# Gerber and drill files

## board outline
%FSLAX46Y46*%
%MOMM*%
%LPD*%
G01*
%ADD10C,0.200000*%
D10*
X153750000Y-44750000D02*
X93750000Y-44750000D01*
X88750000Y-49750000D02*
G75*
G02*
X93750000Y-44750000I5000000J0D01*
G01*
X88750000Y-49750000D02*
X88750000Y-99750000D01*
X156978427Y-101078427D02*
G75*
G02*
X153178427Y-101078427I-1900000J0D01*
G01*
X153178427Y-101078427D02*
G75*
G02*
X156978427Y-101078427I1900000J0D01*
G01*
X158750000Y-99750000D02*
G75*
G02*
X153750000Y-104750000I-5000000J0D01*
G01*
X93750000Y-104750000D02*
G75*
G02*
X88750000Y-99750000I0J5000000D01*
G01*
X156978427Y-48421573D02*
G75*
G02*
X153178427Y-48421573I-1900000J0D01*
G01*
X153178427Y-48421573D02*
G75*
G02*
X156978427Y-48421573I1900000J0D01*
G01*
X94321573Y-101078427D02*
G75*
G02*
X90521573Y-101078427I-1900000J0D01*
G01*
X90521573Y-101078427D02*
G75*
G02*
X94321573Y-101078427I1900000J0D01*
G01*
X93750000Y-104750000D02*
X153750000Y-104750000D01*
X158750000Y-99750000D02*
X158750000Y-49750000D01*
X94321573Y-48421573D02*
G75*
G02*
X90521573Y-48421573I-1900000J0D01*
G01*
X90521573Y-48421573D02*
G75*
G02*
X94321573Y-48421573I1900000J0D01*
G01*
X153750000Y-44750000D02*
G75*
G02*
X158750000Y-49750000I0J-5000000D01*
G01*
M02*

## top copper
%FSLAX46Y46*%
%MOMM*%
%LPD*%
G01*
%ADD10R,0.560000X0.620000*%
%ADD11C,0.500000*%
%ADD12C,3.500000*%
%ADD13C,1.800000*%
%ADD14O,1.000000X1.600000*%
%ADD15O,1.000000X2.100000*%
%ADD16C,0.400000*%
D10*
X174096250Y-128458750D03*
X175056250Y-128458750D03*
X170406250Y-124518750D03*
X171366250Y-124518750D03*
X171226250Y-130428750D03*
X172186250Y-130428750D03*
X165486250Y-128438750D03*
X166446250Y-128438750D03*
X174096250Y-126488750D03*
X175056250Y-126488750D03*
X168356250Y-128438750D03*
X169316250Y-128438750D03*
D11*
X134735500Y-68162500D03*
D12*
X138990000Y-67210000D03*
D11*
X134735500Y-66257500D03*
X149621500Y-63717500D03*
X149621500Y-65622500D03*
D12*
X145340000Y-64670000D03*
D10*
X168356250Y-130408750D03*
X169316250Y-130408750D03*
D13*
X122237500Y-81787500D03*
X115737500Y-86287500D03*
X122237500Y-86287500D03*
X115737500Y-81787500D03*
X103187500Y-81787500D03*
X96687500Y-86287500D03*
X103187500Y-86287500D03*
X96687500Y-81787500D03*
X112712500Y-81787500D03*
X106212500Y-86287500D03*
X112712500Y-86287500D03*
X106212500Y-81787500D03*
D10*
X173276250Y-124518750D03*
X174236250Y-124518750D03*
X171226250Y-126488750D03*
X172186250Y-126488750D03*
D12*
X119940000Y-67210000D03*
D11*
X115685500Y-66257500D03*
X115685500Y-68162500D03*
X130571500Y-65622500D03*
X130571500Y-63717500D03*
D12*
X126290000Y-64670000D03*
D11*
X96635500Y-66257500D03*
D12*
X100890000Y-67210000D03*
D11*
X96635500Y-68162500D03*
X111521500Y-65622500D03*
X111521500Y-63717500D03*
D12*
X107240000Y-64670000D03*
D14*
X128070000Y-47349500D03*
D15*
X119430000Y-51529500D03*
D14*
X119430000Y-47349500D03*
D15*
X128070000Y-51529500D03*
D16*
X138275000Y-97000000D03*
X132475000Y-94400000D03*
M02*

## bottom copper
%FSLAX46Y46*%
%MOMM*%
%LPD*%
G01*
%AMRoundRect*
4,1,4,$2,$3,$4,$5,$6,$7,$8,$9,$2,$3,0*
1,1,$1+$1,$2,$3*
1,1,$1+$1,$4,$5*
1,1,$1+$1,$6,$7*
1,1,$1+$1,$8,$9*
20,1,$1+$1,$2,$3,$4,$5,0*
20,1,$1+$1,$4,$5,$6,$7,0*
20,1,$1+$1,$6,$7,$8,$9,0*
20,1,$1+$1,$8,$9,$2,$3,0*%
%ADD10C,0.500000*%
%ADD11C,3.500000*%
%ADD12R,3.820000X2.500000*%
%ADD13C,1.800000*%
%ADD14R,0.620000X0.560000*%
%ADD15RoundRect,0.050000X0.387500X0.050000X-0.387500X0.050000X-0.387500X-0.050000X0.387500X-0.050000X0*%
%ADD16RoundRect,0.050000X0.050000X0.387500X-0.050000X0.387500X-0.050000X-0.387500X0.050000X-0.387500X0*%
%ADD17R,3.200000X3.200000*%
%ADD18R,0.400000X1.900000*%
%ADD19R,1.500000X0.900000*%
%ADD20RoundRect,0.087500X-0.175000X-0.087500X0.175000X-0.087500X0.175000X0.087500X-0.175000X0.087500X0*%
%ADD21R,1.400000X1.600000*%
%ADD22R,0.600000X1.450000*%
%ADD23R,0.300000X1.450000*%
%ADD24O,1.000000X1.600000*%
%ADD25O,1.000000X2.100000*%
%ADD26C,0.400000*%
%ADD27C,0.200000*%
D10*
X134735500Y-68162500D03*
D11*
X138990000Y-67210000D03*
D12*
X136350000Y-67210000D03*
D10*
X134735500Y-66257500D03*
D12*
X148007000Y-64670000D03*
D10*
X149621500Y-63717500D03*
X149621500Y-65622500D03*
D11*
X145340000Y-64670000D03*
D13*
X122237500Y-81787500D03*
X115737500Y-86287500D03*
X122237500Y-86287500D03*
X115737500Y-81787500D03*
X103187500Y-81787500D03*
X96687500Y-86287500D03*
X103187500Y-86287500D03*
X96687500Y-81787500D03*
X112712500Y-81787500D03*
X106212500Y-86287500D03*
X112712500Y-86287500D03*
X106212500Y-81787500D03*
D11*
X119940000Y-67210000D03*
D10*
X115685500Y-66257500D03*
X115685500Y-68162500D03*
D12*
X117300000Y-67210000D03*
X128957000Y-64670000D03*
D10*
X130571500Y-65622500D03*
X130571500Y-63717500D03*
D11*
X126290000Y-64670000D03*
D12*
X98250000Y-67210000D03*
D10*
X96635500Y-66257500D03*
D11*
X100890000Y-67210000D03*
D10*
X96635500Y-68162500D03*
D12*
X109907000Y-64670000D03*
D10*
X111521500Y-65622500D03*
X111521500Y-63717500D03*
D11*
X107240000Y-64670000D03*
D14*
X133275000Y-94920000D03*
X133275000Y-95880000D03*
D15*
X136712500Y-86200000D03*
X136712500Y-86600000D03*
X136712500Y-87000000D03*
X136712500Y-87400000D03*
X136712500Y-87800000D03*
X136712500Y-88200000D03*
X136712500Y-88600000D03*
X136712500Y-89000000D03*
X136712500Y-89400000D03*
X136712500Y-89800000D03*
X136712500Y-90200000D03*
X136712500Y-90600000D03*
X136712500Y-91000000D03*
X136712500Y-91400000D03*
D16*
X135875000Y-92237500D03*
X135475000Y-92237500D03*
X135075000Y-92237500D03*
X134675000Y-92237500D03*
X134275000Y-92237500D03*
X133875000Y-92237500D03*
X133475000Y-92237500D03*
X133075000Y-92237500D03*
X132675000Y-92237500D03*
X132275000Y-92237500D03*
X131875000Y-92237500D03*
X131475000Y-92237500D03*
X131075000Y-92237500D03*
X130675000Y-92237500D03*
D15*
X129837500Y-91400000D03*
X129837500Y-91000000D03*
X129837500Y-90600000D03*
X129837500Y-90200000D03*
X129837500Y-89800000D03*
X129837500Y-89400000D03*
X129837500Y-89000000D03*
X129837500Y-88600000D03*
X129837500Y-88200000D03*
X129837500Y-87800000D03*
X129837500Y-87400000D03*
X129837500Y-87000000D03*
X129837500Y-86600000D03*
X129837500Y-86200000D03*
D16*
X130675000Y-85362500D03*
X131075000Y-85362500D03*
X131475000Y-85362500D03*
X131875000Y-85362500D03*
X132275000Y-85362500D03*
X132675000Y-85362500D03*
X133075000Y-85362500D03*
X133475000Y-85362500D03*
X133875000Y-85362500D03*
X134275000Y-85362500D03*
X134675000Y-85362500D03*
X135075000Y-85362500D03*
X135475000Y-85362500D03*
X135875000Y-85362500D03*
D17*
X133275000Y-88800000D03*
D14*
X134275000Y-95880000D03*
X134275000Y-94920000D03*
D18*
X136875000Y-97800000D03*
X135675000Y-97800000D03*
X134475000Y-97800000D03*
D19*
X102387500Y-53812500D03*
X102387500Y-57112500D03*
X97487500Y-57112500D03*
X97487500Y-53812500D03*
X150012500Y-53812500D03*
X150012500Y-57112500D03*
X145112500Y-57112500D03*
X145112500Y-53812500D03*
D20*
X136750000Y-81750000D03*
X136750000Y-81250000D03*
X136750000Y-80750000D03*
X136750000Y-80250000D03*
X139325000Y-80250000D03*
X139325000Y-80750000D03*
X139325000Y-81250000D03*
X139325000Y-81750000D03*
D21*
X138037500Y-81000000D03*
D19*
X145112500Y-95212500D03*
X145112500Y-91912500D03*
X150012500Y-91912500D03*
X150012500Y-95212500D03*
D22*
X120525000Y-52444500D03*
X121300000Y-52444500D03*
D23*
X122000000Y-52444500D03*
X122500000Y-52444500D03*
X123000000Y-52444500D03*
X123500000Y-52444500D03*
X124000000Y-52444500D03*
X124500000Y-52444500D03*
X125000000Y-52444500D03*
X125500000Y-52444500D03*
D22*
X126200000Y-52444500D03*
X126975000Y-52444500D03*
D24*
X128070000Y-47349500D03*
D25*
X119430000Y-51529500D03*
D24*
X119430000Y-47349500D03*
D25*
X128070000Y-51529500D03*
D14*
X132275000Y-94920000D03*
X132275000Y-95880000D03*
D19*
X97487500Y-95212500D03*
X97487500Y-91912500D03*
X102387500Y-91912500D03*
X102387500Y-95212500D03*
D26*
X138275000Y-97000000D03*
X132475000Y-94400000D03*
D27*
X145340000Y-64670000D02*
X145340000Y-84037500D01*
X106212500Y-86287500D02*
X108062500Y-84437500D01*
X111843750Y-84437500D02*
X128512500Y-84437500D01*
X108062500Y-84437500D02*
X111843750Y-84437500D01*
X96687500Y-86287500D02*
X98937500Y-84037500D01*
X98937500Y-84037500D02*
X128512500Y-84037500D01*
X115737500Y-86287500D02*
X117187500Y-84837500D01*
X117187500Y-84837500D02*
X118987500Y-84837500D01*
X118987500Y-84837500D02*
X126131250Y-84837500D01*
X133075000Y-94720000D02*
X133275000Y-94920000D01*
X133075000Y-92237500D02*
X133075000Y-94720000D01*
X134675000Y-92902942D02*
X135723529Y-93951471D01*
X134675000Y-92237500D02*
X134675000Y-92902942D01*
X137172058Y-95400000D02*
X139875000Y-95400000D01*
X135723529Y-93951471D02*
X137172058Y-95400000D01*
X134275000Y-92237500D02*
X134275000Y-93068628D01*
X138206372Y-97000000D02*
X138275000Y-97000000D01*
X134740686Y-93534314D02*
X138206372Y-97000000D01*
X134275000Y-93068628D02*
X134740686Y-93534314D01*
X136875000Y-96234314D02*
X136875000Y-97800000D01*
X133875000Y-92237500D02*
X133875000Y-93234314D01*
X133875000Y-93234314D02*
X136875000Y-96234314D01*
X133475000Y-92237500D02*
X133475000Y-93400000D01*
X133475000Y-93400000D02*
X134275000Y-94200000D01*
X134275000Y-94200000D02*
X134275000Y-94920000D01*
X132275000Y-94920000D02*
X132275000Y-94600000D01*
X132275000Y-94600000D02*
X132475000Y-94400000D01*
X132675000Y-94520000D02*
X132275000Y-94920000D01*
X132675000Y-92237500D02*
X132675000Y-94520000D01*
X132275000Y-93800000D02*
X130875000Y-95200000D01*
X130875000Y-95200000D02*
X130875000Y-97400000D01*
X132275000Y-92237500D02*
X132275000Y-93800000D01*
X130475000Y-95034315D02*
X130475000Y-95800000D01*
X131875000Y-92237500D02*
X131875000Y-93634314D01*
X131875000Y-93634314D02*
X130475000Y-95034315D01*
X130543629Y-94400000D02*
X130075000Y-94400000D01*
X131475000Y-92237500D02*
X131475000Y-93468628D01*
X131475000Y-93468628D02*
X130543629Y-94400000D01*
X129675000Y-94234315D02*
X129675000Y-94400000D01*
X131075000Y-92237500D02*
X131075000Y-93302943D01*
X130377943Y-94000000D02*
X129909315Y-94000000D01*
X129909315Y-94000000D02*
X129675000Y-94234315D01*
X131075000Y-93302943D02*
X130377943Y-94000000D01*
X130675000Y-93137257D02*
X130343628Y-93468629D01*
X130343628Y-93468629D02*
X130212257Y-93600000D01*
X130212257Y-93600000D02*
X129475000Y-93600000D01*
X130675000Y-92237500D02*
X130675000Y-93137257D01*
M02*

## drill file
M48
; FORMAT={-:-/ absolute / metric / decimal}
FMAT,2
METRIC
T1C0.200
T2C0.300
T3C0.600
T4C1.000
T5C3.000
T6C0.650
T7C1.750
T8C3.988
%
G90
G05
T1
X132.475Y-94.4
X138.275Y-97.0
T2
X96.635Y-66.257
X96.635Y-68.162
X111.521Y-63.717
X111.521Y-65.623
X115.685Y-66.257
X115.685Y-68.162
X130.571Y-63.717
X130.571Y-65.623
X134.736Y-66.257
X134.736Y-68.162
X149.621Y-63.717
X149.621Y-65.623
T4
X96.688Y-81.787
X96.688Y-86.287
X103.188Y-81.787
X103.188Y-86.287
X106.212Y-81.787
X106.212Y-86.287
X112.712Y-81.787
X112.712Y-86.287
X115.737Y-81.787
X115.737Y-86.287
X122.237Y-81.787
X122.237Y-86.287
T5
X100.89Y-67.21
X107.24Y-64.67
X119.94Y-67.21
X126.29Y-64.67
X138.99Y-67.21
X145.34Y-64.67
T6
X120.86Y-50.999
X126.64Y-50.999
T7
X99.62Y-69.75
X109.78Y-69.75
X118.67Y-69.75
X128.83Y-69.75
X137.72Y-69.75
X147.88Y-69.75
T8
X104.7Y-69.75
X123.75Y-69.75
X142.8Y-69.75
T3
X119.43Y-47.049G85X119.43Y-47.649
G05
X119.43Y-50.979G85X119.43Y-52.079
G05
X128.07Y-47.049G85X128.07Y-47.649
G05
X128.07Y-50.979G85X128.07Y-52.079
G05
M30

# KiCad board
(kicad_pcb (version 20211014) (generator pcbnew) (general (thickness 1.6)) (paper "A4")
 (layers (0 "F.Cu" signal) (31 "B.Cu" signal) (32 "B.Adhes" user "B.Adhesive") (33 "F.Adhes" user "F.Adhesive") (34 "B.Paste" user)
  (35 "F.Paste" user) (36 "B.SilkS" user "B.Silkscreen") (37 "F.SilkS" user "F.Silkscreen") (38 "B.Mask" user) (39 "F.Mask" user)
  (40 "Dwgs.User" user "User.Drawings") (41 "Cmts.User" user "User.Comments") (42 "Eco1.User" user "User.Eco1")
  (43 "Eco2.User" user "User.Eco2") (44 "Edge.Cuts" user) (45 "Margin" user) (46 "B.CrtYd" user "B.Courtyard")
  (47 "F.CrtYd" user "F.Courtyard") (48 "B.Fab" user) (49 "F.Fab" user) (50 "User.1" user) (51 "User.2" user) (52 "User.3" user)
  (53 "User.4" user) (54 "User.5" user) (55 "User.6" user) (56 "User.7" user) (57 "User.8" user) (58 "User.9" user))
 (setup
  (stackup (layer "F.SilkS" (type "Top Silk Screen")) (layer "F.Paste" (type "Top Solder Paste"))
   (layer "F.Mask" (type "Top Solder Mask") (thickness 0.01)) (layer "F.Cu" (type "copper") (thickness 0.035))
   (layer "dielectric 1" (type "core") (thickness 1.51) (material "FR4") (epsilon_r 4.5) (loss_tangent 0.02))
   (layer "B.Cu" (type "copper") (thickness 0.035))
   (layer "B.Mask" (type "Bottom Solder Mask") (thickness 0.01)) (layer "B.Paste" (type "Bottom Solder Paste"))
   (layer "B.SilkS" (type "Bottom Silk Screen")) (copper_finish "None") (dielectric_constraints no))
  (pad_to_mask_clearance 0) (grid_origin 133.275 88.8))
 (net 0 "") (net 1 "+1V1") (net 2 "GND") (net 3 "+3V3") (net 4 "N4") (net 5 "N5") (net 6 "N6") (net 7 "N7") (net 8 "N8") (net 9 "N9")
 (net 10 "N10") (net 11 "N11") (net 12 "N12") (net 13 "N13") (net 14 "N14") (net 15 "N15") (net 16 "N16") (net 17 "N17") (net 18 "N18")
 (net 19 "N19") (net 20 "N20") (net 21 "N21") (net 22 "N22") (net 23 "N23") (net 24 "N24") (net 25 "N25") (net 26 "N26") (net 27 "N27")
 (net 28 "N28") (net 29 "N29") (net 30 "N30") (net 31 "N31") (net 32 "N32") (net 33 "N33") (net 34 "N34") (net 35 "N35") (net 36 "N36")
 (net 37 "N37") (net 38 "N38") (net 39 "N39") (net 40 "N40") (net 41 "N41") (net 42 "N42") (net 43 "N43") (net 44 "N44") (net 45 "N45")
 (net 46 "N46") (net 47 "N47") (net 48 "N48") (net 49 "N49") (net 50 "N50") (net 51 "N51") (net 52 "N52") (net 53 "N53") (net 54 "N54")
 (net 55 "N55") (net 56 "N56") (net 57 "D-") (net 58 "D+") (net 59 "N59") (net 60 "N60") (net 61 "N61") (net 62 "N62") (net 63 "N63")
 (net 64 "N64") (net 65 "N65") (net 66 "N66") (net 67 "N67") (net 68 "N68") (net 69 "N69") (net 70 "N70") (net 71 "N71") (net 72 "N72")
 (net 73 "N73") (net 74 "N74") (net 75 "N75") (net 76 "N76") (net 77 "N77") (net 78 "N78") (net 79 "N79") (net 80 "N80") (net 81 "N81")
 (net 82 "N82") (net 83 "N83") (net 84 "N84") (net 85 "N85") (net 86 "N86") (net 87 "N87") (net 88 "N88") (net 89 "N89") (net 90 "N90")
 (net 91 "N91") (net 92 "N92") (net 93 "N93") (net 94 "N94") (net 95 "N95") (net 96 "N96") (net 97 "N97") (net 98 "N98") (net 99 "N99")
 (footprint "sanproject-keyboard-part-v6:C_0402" (layer "F.Cu") (at 174.57625 128.45875)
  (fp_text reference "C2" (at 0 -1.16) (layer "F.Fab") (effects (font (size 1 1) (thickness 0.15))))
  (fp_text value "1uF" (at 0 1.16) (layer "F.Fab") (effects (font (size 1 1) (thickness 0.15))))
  (pad "1" smd rect locked (at -0.48 0) (size 0.56 0.62) (layers "F.Cu" "F.Paste" "F.Mask") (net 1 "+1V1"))
  (pad "2" smd rect locked (at 0.48 0) (size 0.56 0.62) (layers "F.Cu" "F.Paste" "F.Mask") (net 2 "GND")))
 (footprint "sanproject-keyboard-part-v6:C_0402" (layer "F.Cu") (at 170.88625 124.51875)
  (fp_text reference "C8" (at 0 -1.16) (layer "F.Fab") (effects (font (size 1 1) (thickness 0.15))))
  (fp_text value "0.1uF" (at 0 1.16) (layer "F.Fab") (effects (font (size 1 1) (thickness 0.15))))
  (pad "1" smd rect locked (at -0.48 0) (size 0.56 0.62) (layers "F.Cu" "F.Paste" "F.Mask") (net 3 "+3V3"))
  (pad "2" smd rect locked (at 0.48 0) (size 0.56 0.62) (layers "F.Cu" "F.Paste" "F.Mask") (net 2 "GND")))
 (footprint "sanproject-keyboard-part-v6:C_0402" (layer "F.Cu") (at 171.70625 130.42875)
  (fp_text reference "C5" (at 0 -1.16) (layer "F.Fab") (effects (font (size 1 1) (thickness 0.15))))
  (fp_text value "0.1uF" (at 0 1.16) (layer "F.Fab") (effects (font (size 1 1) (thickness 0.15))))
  (pad "1" smd rect locked (at -0.48 0) (size 0.56 0.62) (layers "F.Cu" "F.Paste" "F.Mask") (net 3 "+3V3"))
  (pad "2" smd rect locked (at 0.48 0) (size 0.56 0.62) (layers "F.Cu" "F.Paste" "F.Mask") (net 2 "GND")))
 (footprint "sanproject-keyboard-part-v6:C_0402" (layer "F.Cu") (at 165.96625 128.43875)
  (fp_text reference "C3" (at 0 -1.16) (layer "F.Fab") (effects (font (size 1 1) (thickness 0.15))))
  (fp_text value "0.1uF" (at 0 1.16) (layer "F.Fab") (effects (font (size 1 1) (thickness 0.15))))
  (pad "1" smd rect locked (at -0.48 0) (size 0.56 0.62) (layers "F.Cu" "F.Paste" "F.Mask") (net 3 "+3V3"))
  (pad "2" smd rect locked (at 0.48 0) (size 0.56 0.62) (layers "F.Cu" "F.Paste" "F.Mask") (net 2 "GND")))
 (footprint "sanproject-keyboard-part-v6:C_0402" (layer "F.Cu") (at 174.57625 126.48875)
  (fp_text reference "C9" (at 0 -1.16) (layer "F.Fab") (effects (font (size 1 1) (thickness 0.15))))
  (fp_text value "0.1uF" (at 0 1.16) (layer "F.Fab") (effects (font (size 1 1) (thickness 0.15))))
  (pad "1" smd rect locked (at -0.48 0) (size 0.56 0.62) (layers "F.Cu" "F.Paste" "F.Mask") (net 3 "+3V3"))
  (pad "2" smd rect locked (at 0.48 0) (size 0.56 0.62) (layers "F.Cu" "F.Paste" "F.Mask") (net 2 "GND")))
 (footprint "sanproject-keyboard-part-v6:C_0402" (layer "F.Cu") (at 168.83625 128.43875)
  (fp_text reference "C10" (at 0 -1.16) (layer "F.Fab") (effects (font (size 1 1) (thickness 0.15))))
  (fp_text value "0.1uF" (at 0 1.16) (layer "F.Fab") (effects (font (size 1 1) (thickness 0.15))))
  (pad "1" smd rect locked (at -0.48 0) (size 0.56 0.62) (layers "F.Cu" "F.Paste" "F.Mask") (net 3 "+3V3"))
  (pad "2" smd rect locked (at 0.48 0) (size 0.56 0.62) (layers "F.Cu" "F.Paste" "F.Mask") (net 2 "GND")))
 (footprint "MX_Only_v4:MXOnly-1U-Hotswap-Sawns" (layer "F.Cu") (at 142.8 69.75)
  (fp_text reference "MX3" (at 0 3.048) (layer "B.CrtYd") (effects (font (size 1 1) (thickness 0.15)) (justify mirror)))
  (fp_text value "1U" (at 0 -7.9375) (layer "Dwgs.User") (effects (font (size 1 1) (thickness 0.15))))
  (pad "" np_thru_hole circle locked (at 5.08 0 48.0996) (size 1.75 1.75) (drill 1.75) (layers *.Cu *.Mask))
  (pad "" smd rect locked (at 5.842 -5.08) (size 2.55 2.5) (layers "B.Paste" "B.Mask"))
  (pad "" np_thru_hole circle locked (at -5.08 0 48.0996) (size 1.75 1.75) (drill 1.75) (layers *.Cu *.Mask))
  (pad "" smd rect locked (at -7.085 -2.54) (size 2.55 2.5) (layers "B.Paste" "B.Mask"))
  (pad "" np_thru_hole circle locked (at 0 0) (size 3.9878 3.9878) (drill 3.9878) (layers *.Cu *.Mask))
  (pad "1" thru_hole circle locked (at -8.0645 -1.5875) (size 0.5 0.5) (drill 0.3) (layers *.Cu *.Mask) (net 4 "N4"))
  (pad "1" thru_hole circle locked (at -3.81 -2.54) (size 3.5 3.5) (drill 3) (layers *.Cu *.Mask) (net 4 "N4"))
  (pad "1" smd rect locked (at -6.45 -2.54) (size 3.82 2.5) (layers "B.Cu") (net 4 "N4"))
  (pad "1" thru_hole circle locked (at -8.0645 -3.4925) (size 0.5 0.5) (drill 0.3) (layers *.Cu *.Mask) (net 4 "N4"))
  (pad "2" smd rect locked (at 5.207 -5.08) (size 3.82 2.5) (layers "B.Cu") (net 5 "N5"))
  (pad "2" thru_hole circle locked (at 6.8215 -6.0325) (size 0.5 0.5) (drill 0.3) (layers *.Cu *.Mask) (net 5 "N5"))
  (pad "2" thru_hole circle locked (at 6.8215 -4.1275) (size 0.5 0.5) (drill 0.3) (layers *.Cu *.Mask) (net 5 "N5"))
  (pad "2" thru_hole circle locked (at 2.54 -5.08) (size 3.5 3.5) (drill 3) (layers *.Cu *.Mask) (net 5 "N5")))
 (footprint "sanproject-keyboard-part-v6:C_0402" (layer "F.Cu") (at 168.83625 130.40875)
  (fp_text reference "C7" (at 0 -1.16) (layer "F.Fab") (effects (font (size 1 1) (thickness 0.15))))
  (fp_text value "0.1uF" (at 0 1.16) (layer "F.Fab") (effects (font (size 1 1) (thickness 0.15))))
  (pad "1" smd rect locked (at -0.48 0) (size 0.56 0.62) (layers "F.Cu" "F.Paste" "F.Mask") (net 3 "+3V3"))
  (pad "2" smd rect locked (at 0.48 0) (size 0.56 0.62) (layers "F.Cu" "F.Paste" "F.Mask") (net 2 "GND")))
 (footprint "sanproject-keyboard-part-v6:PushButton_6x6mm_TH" (layer "F.Cu") (at 118.9875 84.0375)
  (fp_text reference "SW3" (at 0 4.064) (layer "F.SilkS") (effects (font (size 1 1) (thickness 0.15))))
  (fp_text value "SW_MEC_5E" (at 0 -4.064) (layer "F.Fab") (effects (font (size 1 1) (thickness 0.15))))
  (pad "1" thru_hole circle locked (at 3.25 -2.25) (size 1.8 1.8) (drill 1) (layers *.Cu *.Mask) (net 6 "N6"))
  (pad "2" thru_hole circle locked (at -3.25 2.25) (size 1.8 1.8) (drill 1) (layers *.Cu *.Mask) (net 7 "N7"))
  (pad "3" thru_hole circle locked (at 3.25 2.25) (size 1.8 1.8) (drill 1) (layers *.Cu *.Mask) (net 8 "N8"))
  (pad "4" thru_hole circle locked (at -3.25 -2.25) (size 1.8 1.8) (drill 1) (layers *.Cu *.Mask) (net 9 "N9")))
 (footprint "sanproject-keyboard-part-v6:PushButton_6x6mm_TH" (layer "F.Cu") (at 99.9375 84.0375)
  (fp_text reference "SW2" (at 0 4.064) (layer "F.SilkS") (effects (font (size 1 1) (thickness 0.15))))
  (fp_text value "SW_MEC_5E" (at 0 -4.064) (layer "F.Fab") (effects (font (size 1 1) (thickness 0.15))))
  (pad "1" thru_hole circle locked (at 3.25 -2.25) (size 1.8 1.8) (drill 1) (layers *.Cu *.Mask) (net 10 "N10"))
  (pad "2" thru_hole circle locked (at -3.25 2.25) (size 1.8 1.8) (drill 1) (layers *.Cu *.Mask) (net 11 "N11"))
  (pad "3" thru_hole circle locked (at 3.25 2.25) (size 1.8 1.8) (drill 1) (layers *.Cu *.Mask) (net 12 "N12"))
  (pad "4" thru_hole circle locked (at -3.25 -2.25) (size 1.8 1.8) (drill 1) (layers *.Cu *.Mask) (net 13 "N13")))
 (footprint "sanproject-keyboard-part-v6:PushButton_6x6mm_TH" (layer "F.Cu") (at 109.4625 84.0375)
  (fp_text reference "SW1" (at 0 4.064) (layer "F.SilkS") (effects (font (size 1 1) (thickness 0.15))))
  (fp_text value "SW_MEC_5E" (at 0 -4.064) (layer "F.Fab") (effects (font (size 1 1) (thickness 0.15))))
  (pad "1" thru_hole circle locked (at 3.25 -2.25) (size 1.8 1.8) (drill 1) (layers *.Cu *.Mask) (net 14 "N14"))
  (pad "2" thru_hole circle locked (at -3.25 2.25) (size 1.8 1.8) (drill 1) (layers *.Cu *.Mask) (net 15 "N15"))
  (pad "3" thru_hole circle locked (at 3.25 2.25) (size 1.8 1.8) (drill 1) (layers *.Cu *.Mask) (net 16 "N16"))
  (pad "4" thru_hole circle locked (at -3.25 -2.25) (size 1.8 1.8) (drill 1) (layers *.Cu *.Mask) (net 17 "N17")))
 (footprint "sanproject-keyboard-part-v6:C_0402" (layer "F.Cu") (at 173.75625 124.51875)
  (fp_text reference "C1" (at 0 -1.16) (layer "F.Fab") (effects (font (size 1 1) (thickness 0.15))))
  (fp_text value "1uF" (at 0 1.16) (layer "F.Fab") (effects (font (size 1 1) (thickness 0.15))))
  (pad "1" smd rect locked (at -0.48 0) (size 0.56 0.62) (layers "F.Cu" "F.Paste" "F.Mask") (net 3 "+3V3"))
  (pad "2" smd rect locked (at 0.48 0) (size 0.56 0.62) (layers "F.Cu" "F.Paste" "F.Mask") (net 2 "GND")))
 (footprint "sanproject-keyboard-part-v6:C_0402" (layer "F.Cu") (at 171.70625 126.48875)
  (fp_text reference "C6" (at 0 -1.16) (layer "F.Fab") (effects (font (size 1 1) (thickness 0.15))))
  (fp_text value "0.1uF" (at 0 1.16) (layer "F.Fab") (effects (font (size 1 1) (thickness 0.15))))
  (pad "1" smd rect locked (at -0.48 0) (size 0.56 0.62) (layers "F.Cu" "F.Paste" "F.Mask") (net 1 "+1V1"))
  (pad "2" smd rect locked (at 0.48 0) (size 0.56 0.62) (layers "F.Cu" "F.Paste" "F.Mask") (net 2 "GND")))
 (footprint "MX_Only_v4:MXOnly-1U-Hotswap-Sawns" (layer "F.Cu") (at 123.75 69.75)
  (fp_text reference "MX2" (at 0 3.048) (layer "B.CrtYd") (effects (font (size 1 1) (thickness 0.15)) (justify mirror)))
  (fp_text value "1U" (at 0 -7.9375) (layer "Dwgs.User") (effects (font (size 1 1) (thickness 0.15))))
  (pad "" np_thru_hole circle locked (at -5.08 0 48.0996) (size 1.75 1.75) (drill 1.75) (layers *.Cu *.Mask))
  (pad "" np_thru_hole circle locked (at 0 0) (size 3.9878 3.9878) (drill 3.9878) (layers *.Cu *.Mask))
  (pad "" np_thru_hole circle locked (at 5.08 0 48.0996) (size 1.75 1.75) (drill 1.75) (layers *.Cu *.Mask))
  (pad "" smd rect locked (at -7.085 -2.54) (size 2.55 2.5) (layers "B.Paste" "B.Mask"))
  (pad "" smd rect locked (at 5.842 -5.08) (size 2.55 2.5) (layers "B.Paste" "B.Mask"))
  (pad "1" thru_hole circle locked (at -3.81 -2.54) (size 3.5 3.5) (drill 3) (layers *.Cu *.Mask) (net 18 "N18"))
  (pad "1" thru_hole circle locked (at -8.0645 -3.4925) (size 0.5 0.5) (drill 0.3) (layers *.Cu *.Mask) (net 18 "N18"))
  (pad "1" thru_hole circle locked (at -8.0645 -1.5875) (size 0.5 0.5) (drill 0.3) (layers *.Cu *.Mask) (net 18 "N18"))
  (pad "1" smd rect locked (at -6.45 -2.54) (size 3.82 2.5) (layers "B.Cu") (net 18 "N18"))
  (pad "2" smd rect locked (at 5.207 -5.08) (size 3.82 2.5) (layers "B.Cu") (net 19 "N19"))
  (pad "2" thru_hole circle locked (at 6.8215 -4.1275) (size 0.5 0.5) (drill 0.3) (layers *.Cu *.Mask) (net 19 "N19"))
  (pad "2" thru_hole circle locked (at 6.8215 -6.0325) (size 0.5 0.5) (drill 0.3) (layers *.Cu *.Mask) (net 19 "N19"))
  (pad "2" thru_hole circle locked (at 2.54 -5.08) (size 3.5 3.5) (drill 3) (layers *.Cu *.Mask) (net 19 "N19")))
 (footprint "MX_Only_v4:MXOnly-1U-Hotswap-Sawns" (layer "F.Cu") (at 104.7 69.75)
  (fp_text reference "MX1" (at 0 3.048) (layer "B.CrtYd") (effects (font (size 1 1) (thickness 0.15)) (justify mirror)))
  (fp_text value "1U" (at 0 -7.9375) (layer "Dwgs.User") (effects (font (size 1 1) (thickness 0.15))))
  (pad "" np_thru_hole circle locked (at -5.08 0 48.0996) (size 1.75 1.75) (drill 1.75) (layers *.Cu *.Mask))
  (pad "" np_thru_hole circle locked (at 5.08 0 48.0996) (size 1.75 1.75) (drill 1.75) (layers *.Cu *.Mask))
  (pad "" smd rect locked (at -7.085 -2.54) (size 2.55 2.5) (layers "B.Paste" "B.Mask"))
  (pad "" smd rect locked (at 5.842 -5.08) (size 2.55 2.5) (layers "B.Paste" "B.Mask"))
  (pad "" np_thru_hole circle locked (at 0 0) (size 3.9878 3.9878) (drill 3.9878) (layers *.Cu *.Mask))
  (pad "1" smd rect locked (at -6.45 -2.54) (size 3.82 2.5) (layers "B.Cu") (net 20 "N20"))
  (pad "1" thru_hole circle locked (at -8.0645 -3.4925) (size 0.5 0.5) (drill 0.3) (layers *.Cu *.Mask) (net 20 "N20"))
  (pad "1" thru_hole circle locked (at -3.81 -2.54) (size 3.5 3.5) (drill 3) (layers *.Cu *.Mask) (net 20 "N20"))
  (pad "1" thru_hole circle locked (at -8.0645 -1.5875) (size 0.5 0.5) (drill 0.3) (layers *.Cu *.Mask) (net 20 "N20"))
  (pad "2" smd rect locked (at 5.207 -5.08) (size 3.82 2.5) (layers "B.Cu") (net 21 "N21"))
  (pad "2" thru_hole circle locked (at 6.8215 -4.1275) (size 0.5 0.5) (drill 0.3) (layers *.Cu *.Mask) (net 21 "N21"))
  (pad "2" thru_hole circle locked (at 6.8215 -6.0325) (size 0.5 0.5) (drill 0.3) (layers *.Cu *.Mask) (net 21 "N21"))
  (pad "2" thru_hole circle locked (at 2.54 -5.08) (size 3.5 3.5) (drill 3) (layers *.Cu *.Mask) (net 21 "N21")))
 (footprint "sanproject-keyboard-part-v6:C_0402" (layer "B.Cu") (at 133.275 95.4 -90)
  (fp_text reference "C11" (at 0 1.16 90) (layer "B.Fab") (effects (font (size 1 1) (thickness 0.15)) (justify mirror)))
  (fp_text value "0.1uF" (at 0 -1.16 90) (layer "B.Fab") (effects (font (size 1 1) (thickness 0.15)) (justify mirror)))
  (pad "1" smd rect locked (at -0.48 0 270) (size 0.56 0.62) (layers "B.Cu" "B.Paste" "B.Mask") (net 3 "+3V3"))
  (pad "2" smd rect locked (at 0.48 0 270) (size 0.56 0.62) (layers "B.Cu" "B.Paste" "B.Mask") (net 2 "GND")))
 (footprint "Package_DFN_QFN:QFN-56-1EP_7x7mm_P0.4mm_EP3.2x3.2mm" (layer "B.Cu") (at 133.275 88.8 180)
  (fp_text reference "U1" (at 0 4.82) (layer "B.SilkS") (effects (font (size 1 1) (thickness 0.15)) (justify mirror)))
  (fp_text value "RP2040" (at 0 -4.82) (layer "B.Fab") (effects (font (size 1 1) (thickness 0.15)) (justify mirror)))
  (pad "" smd roundrect locked (at -0.8 0.8 180) (size 1.29 1.29) (layers "B.Paste") (roundrect_rratio 0.193798))
  (pad "" smd roundrect locked (at -0.8 -0.8 180) (size 1.29 1.29) (layers "B.Paste") (roundrect_rratio 0.193798))
  (pad "" smd roundrect locked (at 0.8 0.8 180) (size 1.29 1.29) (layers "B.Paste") (roundrect_rratio 0.193798))
  (pad "" smd roundrect locked (at 0.8 -0.8 180) (size 1.29 1.29) (layers "B.Paste") (roundrect_rratio 0.193798))
  (pad "1" smd roundrect locked (at -3.4375 2.6 180) (size 0.875 0.2) (layers "B.Cu" "B.Paste" "B.Mask") (roundrect_rratio 0.25)
   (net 3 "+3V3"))
  (pad "2" smd roundrect locked (at -3.4375 2.2 180) (size 0.875 0.2) (layers "B.Cu" "B.Paste" "B.Mask") (roundrect_rratio 0.25)
   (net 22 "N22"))
  (pad "3" smd roundrect locked (at -3.4375 1.8 180) (size 0.875 0.2) (layers "B.Cu" "B.Paste" "B.Mask") (roundrect_rratio 0.25)
   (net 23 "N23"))
  (pad "4" smd roundrect locked (at -3.4375 1.4 180) (size 0.875 0.2) (layers "B.Cu" "B.Paste" "B.Mask") (roundrect_rratio 0.25)
   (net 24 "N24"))
  (pad "5" smd roundrect locked (at -3.4375 1 180) (size 0.875 0.2) (layers "B.Cu" "B.Paste" "B.Mask") (roundrect_rratio 0.25)
   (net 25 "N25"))
  (pad "6" smd roundrect locked (at -3.4375 0.6 180) (size 0.875 0.2) (layers "B.Cu" "B.Paste" "B.Mask") (roundrect_rratio 0.25)
   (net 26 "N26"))
  (pad "7" smd roundrect locked (at -3.4375 0.2 180) (size 0.875 0.2) (layers "B.Cu" "B.Paste" "B.Mask") (roundrect_rratio 0.25)
   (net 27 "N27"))
  (pad "8" smd roundrect locked (at -3.4375 -0.2 180) (size 0.875 0.2) (layers "B.Cu" "B.Paste" "B.Mask") (roundrect_rratio 0.25)
   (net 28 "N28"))
  (pad "9" smd roundrect locked (at -3.4375 -0.6 180) (size 0.875 0.2) (layers "B.Cu" "B.Paste" "B.Mask") (roundrect_rratio 0.25)
   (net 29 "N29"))
  (pad "10" smd roundrect locked (at -3.4375 -1 180) (size 0.875 0.2) (layers "B.Cu" "B.Paste" "B.Mask") (roundrect_rratio 0.25)
   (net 3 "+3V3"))
  (pad "11" smd roundrect locked (at -3.4375 -1.4 180) (size 0.875 0.2) (layers "B.Cu" "B.Paste" "B.Mask") (roundrect_rratio 0.25)
   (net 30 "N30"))
  (pad "12" smd roundrect locked (at -3.4375 -1.8 180) (size 0.875 0.2) (layers "B.Cu" "B.Paste" "B.Mask") (roundrect_rratio 0.25)
   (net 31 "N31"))
  (pad "13" smd roundrect locked (at -3.4375 -2.2 180) (size 0.875 0.2) (layers "B.Cu" "B.Paste" "B.Mask") (roundrect_rratio 0.25)
   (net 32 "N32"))
  (pad "14" smd roundrect locked (at -3.4375 -2.6 180) (size 0.875 0.2) (layers "B.Cu" "B.Paste" "B.Mask") (roundrect_rratio 0.25)
   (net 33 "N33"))
  (pad "15" smd roundrect locked (at -2.6 -3.4375 180) (size 0.2 0.875) (layers "B.Cu" "B.Paste" "B.Mask") (roundrect_rratio 0.25)
   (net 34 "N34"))
  (pad "16" smd roundrect locked (at -2.2 -3.4375 180) (size 0.2 0.875) (layers "B.Cu" "B.Paste" "B.Mask") (roundrect_rratio 0.25)
   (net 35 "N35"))
  (pad "17" smd roundrect locked (at -1.8 -3.4375 180) (size 0.2 0.875) (layers "B.Cu" "B.Paste" "B.Mask") (roundrect_rratio 0.25)
   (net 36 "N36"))
  (pad "18" smd roundrect locked (at -1.4 -3.4375 180) (size 0.2 0.875) (layers "B.Cu" "B.Paste" "B.Mask") (roundrect_rratio 0.25)
   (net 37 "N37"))
  (pad "19" smd roundrect locked (at -1 -3.4375 180) (size 0.2 0.875) (layers "B.Cu" "B.Paste" "B.Mask") (roundrect_rratio 0.25)
   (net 2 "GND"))
  (pad "20" smd roundrect locked (at -0.6 -3.4375 180) (size 0.2 0.875) (layers "B.Cu" "B.Paste" "B.Mask") (roundrect_rratio 0.25)
   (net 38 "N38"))
  (pad "21" smd roundrect locked (at -0.2 -3.4375 180) (size 0.2 0.875) (layers "B.Cu" "B.Paste" "B.Mask") (roundrect_rratio 0.25)
   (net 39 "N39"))
  (pad "22" smd roundrect locked (at 0.2 -3.4375 180) (size 0.2 0.875) (layers "B.Cu" "B.Paste" "B.Mask") (roundrect_rratio 0.25)
   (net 3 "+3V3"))
  (pad "23" smd roundrect locked (at 0.6 -3.4375 180) (size 0.2 0.875) (layers "B.Cu" "B.Paste" "B.Mask") (roundrect_rratio 0.25)
   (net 1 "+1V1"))
  (pad "24" smd roundrect locked (at 1 -3.4375 180) (size 0.2 0.875) (layers "B.Cu" "B.Paste" "B.Mask") (roundrect_rratio 0.25)
   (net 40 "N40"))
  (pad "25" smd roundrect locked (at 1.4 -3.4375 180) (size 0.2 0.875) (layers "B.Cu" "B.Paste" "B.Mask") (roundrect_rratio 0.25)
   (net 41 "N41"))
  (pad "26" smd roundrect locked (at 1.8 -3.4375 180) (size 0.2 0.875) (layers "B.Cu" "B.Paste" "B.Mask") (roundrect_rratio 0.25)
   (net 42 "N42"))
  (pad "27" smd roundrect locked (at 2.2 -3.4375 180) (size 0.2 0.875) (layers "B.Cu" "B.Paste" "B.Mask") (roundrect_rratio 0.25)
   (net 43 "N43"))
  (pad "28" smd roundrect locked (at 2.6 -3.4375 180) (size 0.2 0.875) (layers "B.Cu" "B.Paste" "B.Mask") (roundrect_rratio 0.25)
   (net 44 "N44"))
  (pad "29" smd roundrect locked (at 3.4375 -2.6 180) (size 0.875 0.2) (layers "B.Cu" "B.Paste" "B.Mask") (roundrect_rratio 0.25)
   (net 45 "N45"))
  (pad "30" smd roundrect locked (at 3.4375 -2.2 180) (size 0.875 0.2) (layers "B.Cu" "B.Paste" "B.Mask") (roundrect_rratio 0.25)
   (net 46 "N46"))
  (pad "31" smd roundrect locked (at 3.4375 -1.8 180) (size 0.875 0.2) (layers "B.Cu" "B.Paste" "B.Mask") (roundrect_rratio 0.25)
   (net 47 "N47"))
  (pad "32" smd roundrect locked (at 3.4375 -1.4 180) (size 0.875 0.2) (layers "B.Cu" "B.Paste" "B.Mask") (roundrect_rratio 0.25)
   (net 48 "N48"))
  (pad "33" smd roundrect locked (at 3.4375 -1 180) (size 0.875 0.2) (layers "B.Cu" "B.Paste" "B.Mask") (roundrect_rratio 0.25)
   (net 3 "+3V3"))
  (pad "34" smd roundrect locked (at 3.4375 -0.6 180) (size 0.875 0.2) (layers "B.Cu" "B.Paste" "B.Mask") (roundrect_rratio 0.25)
   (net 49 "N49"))
  (pad "35" smd roundrect locked (at 3.4375 -0.2 180) (size 0.875 0.2) (layers "B.Cu" "B.Paste" "B.Mask") (roundrect_rratio 0.25)
   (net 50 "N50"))
  (pad "36" smd roundrect locked (at 3.4375 0.2 180) (size 0.875 0.2) (layers "B.Cu" "B.Paste" "B.Mask") (roundrect_rratio 0.25)
   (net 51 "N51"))
  (pad "37" smd roundrect locked (at 3.4375 0.6 180) (size 0.875 0.2) (layers "B.Cu" "B.Paste" "B.Mask") (roundrect_rratio 0.25)
   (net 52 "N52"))
  (pad "38" smd roundrect locked (at 3.4375 1 180) (size 0.875 0.2) (layers "B.Cu" "B.Paste" "B.Mask") (roundrect_rratio 0.25)
   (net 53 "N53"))
  (pad "39" smd roundrect locked (at 3.4375 1.4 180) (size 0.875 0.2) (layers "B.Cu" "B.Paste" "B.Mask") (roundrect_rratio 0.25)
   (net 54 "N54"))
  (pad "40" smd roundrect locked (at 3.4375 1.8 180) (size 0.875 0.2) (layers "B.Cu" "B.Paste" "B.Mask") (roundrect_rratio 0.25)
   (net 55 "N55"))
  (pad "41" smd roundrect locked (at 3.4375 2.2 180) (size 0.875 0.2) (layers "B.Cu" "B.Paste" "B.Mask") (roundrect_rratio 0.25)
   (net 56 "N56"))
  (pad "42" smd roundrect locked (at 3.4375 2.6 180) (size 0.875 0.2) (layers "B.Cu" "B.Paste" "B.Mask") (roundrect_rratio 0.25)
   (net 3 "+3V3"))
  (pad "43" smd roundrect locked (at 2.6 3.4375 180) (size 0.2 0.875) (layers "B.Cu" "B.Paste" "B.Mask") (roundrect_rratio 0.25)
   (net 3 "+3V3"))
  (pad "44" smd roundrect locked (at 2.2 3.4375 180) (size 0.2 0.875) (layers "B.Cu" "B.Paste" "B.Mask") (roundrect_rratio 0.25)
   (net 3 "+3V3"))
  (pad "45" smd roundrect locked (at 1.8 3.4375 180) (size 0.2 0.875) (layers "B.Cu" "B.Paste" "B.Mask") (roundrect_rratio 0.25)
   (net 1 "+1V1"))
  (pad "46" smd roundrect locked (at 1.4 3.4375 180) (size 0.2 0.875) (layers "B.Cu" "B.Paste" "B.Mask") (roundrect_rratio 0.25)
   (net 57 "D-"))
  (pad "47" smd roundrect locked (at 1 3.4375 180) (size 0.2 0.875) (layers "B.Cu" "B.Paste" "B.Mask") (roundrect_rratio 0.25) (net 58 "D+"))
  (pad "48" smd roundrect locked (at 0.6 3.4375 180) (size 0.2 0.875) (layers "B.Cu" "B.Paste" "B.Mask") (roundrect_rratio 0.25)
   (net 3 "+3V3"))
  (pad "49" smd roundrect locked (at 0.2 3.4375 180) (size 0.2 0.875) (layers "B.Cu" "B.Paste" "B.Mask") (roundrect_rratio 0.25)
   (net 3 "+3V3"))
  (pad "50" smd roundrect locked (at -0.2 3.4375 180) (size 0.2 0.875) (layers "B.Cu" "B.Paste" "B.Mask") (roundrect_rratio 0.25)
   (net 1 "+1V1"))
  (pad "51" smd roundrect locked (at -0.6 3.4375 180) (size 0.2 0.875) (layers "B.Cu" "B.Paste" "B.Mask") (roundrect_rratio 0.25)
   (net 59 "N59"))
  (pad "52" smd roundrect locked (at -1 3.4375 180) (size 0.2 0.875) (layers "B.Cu" "B.Paste" "B.Mask") (roundrect_rratio 0.25)
   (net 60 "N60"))
  (pad "53" smd roundrect locked (at -1.4 3.4375 180) (size 0.2 0.875) (layers "B.Cu" "B.Paste" "B.Mask") (roundrect_rratio 0.25)
   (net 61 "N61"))
  (pad "54" smd roundrect locked (at -1.8 3.4375 180) (size 0.2 0.875) (layers "B.Cu" "B.Paste" "B.Mask") (roundrect_rratio 0.25)
   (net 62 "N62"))
  (pad "55" smd roundrect locked (at -2.2 3.4375 180) (size 0.2 0.875) (layers "B.Cu" "B.Paste" "B.Mask") (roundrect_rratio 0.25)
   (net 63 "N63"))
  (pad "56" smd roundrect locked (at -2.6 3.4375 180) (size 0.2 0.875) (layers "B.Cu" "B.Paste" "B.Mask") (roundrect_rratio 0.25)
   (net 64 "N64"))
  (pad "57" smd rect locked (at 0 0 180) (size 3.2 3.2) (layers "B.Cu" "B.Mask") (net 2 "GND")))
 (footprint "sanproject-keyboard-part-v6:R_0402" (layer "B.Cu") (at 134.275 95.4 90)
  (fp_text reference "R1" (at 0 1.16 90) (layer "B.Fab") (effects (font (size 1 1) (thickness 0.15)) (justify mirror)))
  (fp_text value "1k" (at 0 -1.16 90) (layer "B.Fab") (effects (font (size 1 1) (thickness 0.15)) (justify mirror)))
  (pad "1" smd rect locked (at -0.48 0 90) (size 0.56 0.62) (layers "B.Cu" "B.Paste" "B.Mask") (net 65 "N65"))
  (pad "2" smd rect locked (at 0.48 0 90) (size 0.56 0.62) (layers "B.Cu" "B.Paste" "B.Mask") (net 39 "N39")))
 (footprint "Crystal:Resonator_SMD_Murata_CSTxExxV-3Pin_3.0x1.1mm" (layer "B.Cu") (at 135.675 97.8 180)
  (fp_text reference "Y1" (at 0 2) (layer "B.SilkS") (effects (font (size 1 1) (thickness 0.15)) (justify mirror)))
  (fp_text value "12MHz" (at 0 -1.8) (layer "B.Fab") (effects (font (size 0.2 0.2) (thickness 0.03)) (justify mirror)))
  (pad "1" smd rect (at -1.2 0 180) (size 0.4 1.9) (layers "B.Cu" "B.Paste" "B.Mask") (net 38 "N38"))
  (pad "2" smd rect (at 0 0 180) (size 0.4 1.9) (layers "B.Cu" "B.Paste" "B.Mask") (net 2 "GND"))
  (pad "3" smd rect (at 1.2 0 180) (size 0.4 1.9) (layers "B.Cu" "B.Paste" "B.Mask") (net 65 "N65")))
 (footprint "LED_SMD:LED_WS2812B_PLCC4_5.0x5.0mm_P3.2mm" (layer "B.Cu") (at 99.9375 55.4625 180)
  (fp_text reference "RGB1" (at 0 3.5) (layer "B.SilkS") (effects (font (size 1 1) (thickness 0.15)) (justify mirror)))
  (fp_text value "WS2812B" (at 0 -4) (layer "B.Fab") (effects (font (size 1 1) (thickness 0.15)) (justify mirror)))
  (pad "1" smd rect (at -2.45 1.65 180) (size 1.5 0.9) (layers "B.Cu" "B.Paste" "B.Mask") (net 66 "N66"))
  (pad "2" smd rect (at -2.45 -1.65 180) (size 1.5 0.9) (layers "B.Cu" "B.Paste" "B.Mask") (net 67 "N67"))
  (pad "3" smd rect (at 2.45 -1.65 180) (size 1.5 0.9) (layers "B.Cu" "B.Paste" "B.Mask") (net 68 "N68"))
  (pad "4" smd rect (at 2.45 1.65 180) (size 1.5 0.9) (layers "B.Cu" "B.Paste" "B.Mask") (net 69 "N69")))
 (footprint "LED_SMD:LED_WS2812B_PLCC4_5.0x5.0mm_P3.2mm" (layer "B.Cu") (at 147.5625 55.4625 180)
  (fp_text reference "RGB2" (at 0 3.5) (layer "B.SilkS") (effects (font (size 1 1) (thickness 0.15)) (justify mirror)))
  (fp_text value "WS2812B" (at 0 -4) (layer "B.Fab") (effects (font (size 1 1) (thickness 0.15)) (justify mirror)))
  (pad "1" smd rect (at -2.45 1.65 180) (size 1.5 0.9) (layers "B.Cu" "B.Paste" "B.Mask") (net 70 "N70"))
  (pad "2" smd rect (at -2.45 -1.65 180) (size 1.5 0.9) (layers "B.Cu" "B.Paste" "B.Mask") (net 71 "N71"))
  (pad "3" smd rect (at 2.45 -1.65 180) (size 1.5 0.9) (layers "B.Cu" "B.Paste" "B.Mask") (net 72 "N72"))
  (pad "4" smd rect (at 2.45 1.65 180) (size 1.5 0.9) (layers "B.Cu" "B.Paste" "B.Mask") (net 67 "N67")))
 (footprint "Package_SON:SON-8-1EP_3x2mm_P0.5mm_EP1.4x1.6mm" (layer "B.Cu") (at 138.0375 81)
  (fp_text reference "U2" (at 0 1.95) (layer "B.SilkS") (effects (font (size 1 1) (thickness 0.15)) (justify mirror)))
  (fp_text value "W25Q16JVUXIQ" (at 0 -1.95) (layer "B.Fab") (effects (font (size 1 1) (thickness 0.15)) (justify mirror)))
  (pad "" smd roundrect (at 0.35 0.4) (size 0.56 0.64) (layers "B.Paste") (roundrect_rratio 0.25))
  (pad "" smd roundrect (at -0.35 0.4) (size 0.56 0.64) (layers "B.Paste") (roundrect_rratio 0.25))
  (pad "" smd roundrect (at 0.35 -0.4) (size 0.56 0.64) (layers "B.Paste") (roundrect_rratio 0.25))
  (pad "" smd roundrect (at -0.35 -0.4) (size 0.56 0.64) (layers "B.Paste") (roundrect_rratio 0.25))
  (pad "1" smd roundrect (at -1.2875 0.75) (size 0.525 0.35) (layers "B.Cu" "B.Paste" "B.Mask") (roundrect_rratio 0.25) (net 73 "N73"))
  (pad "2" smd roundrect (at -1.2875 0.25) (size 0.525 0.35) (layers "B.Cu" "B.Paste" "B.Mask") (roundrect_rratio 0.25) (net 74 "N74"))
  (pad "3" smd roundrect (at -1.2875 -0.25) (size 0.525 0.35) (layers "B.Cu" "B.Paste" "B.Mask") (roundrect_rratio 0.25) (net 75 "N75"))
  (pad "4" smd roundrect (at -1.2875 -0.75) (size 0.525 0.35) (layers "B.Cu" "B.Paste" "B.Mask") (roundrect_rratio 0.25) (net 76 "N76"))
  (pad "5" smd roundrect (at 1.2875 -0.75) (size 0.525 0.35) (layers "B.Cu" "B.Paste" "B.Mask") (roundrect_rratio 0.25) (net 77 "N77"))
  (pad "6" smd roundrect (at 1.2875 -0.25) (size 0.525 0.35) (layers "B.Cu" "B.Paste" "B.Mask") (roundrect_rratio 0.25) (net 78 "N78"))
  (pad "7" smd roundrect (at 1.2875 0.25) (size 0.525 0.35) (layers "B.Cu" "B.Paste" "B.Mask") (roundrect_rratio 0.25) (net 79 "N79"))
  (pad "8" smd roundrect (at 1.2875 0.75) (size 0.525 0.35) (layers "B.Cu" "B.Paste" "B.Mask") (roundrect_rratio 0.25) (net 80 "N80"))
  (pad "9" smd rect (at 0 0) (size 1.4 1.6) (layers "B.Cu" "B.Mask")))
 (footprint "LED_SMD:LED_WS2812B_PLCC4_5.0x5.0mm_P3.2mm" (layer "B.Cu") (at 147.5625 93.5625)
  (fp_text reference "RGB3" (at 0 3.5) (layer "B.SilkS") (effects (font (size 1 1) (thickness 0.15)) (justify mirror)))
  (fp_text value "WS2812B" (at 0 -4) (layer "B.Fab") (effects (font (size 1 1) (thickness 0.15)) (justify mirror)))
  (pad "1" smd rect (at -2.45 1.65) (size 1.5 0.9) (layers "B.Cu" "B.Paste" "B.Mask") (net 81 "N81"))
  (pad "2" smd rect (at -2.45 -1.65) (size 1.5 0.9) (layers "B.Cu" "B.Paste" "B.Mask") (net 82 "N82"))
  (pad "3" smd rect (at 2.45 -1.65) (size 1.5 0.9) (layers "B.Cu" "B.Paste" "B.Mask") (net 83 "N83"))
  (pad "4" smd rect (at 2.45 1.65) (size 1.5 0.9) (layers "B.Cu" "B.Paste" "B.Mask") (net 71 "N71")))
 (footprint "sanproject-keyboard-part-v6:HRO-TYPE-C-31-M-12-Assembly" (layer "B.Cu") (at 123.75 44.7495)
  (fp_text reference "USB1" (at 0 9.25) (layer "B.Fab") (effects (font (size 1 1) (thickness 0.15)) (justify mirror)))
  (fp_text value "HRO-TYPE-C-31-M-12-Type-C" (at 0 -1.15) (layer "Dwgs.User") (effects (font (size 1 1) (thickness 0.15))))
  (pad "" np_thru_hole circle locked (at 2.89 6.25) (size 0.65 0.65) (drill 0.65) (layers *.Cu *.Mask))
  (pad "" np_thru_hole circle locked (at -2.89 6.25) (size 0.65 0.65) (drill 0.65) (layers *.Cu *.Mask))
  (pad "1" smd rect locked (at -3.225 7.695) (size 0.6 1.45) (layers "B.Cu" "B.Paste" "B.Mask") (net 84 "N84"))
  (pad "2" smd rect locked (at -2.45 7.695) (size 0.6 1.45) (layers "B.Cu" "B.Paste" "B.Mask") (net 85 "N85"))
  (pad "3" smd rect locked (at -1.75 7.695) (size 0.3 1.45) (layers "B.Cu" "B.Paste" "B.Mask") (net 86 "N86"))
  (pad "4" smd rect locked (at -1.25 7.695) (size 0.3 1.45) (layers "B.Cu" "B.Paste" "B.Mask") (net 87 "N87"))
  (pad "5" smd rect locked (at -0.75 7.695) (size 0.3 1.45) (layers "B.Cu" "B.Paste" "B.Mask") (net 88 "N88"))
  (pad "6" smd rect locked (at -0.25 7.695) (size 0.3 1.45) (layers "B.Cu" "B.Paste" "B.Mask") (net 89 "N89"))
  (pad "7" smd rect locked (at 0.25 7.695) (size 0.3 1.45) (layers "B.Cu" "B.Paste" "B.Mask") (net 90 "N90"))
  (pad "8" smd rect locked (at 0.75 7.695) (size 0.3 1.45) (layers "B.Cu" "B.Paste" "B.Mask") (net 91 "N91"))
  (pad "9" smd rect locked (at 1.25 7.695) (size 0.3 1.45) (layers "B.Cu" "B.Paste" "B.Mask") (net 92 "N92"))
  (pad "10" smd rect locked (at 1.75 7.695) (size 0.3 1.45) (layers "B.Cu" "B.Paste" "B.Mask") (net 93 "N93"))
  (pad "11" smd rect locked (at 2.45 7.695) (size 0.6 1.45) (layers "B.Cu" "B.Paste" "B.Mask") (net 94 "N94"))
  (pad "12" smd rect locked (at 3.225 7.695) (size 0.6 1.45) (layers "B.Cu" "B.Paste" "B.Mask") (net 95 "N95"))
  (pad "13" thru_hole oval locked (at 4.32 2.6) (size 1 1.6) (drill oval 0.6 1.2) (layers *.Cu *.Mask "B.Paste") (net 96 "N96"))
  (pad "13" thru_hole oval locked (at -4.32 6.78) (size 1 2.1) (drill oval 0.6 1.7) (layers *.Cu *.Mask "B.Paste") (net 96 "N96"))
  (pad "13" thru_hole oval locked (at -4.32 2.6) (size 1 1.6) (drill oval 0.6 1.2) (layers *.Cu *.Mask "B.Paste") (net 96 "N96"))
  (pad "13" thru_hole oval locked (at 4.32 6.78) (size 1 2.1) (drill oval 0.6 1.7) (layers *.Cu *.Mask "B.Paste") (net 96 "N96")))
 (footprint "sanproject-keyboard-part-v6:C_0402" (layer "B.Cu") (at 132.275 95.4 -90)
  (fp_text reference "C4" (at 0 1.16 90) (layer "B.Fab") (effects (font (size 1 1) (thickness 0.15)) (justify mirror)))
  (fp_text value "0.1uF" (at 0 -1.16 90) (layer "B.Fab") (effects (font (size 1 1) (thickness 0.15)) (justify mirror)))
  (pad "1" smd rect locked (at -0.48 0 270) (size 0.56 0.62) (layers "B.Cu" "B.Paste" "B.Mask") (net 1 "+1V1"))
  (pad "2" smd rect locked (at 0.48 0 270) (size 0.56 0.62) (layers "B.Cu" "B.Paste" "B.Mask") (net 2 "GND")))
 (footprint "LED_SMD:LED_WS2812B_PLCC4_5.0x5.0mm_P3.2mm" (layer "B.Cu") (at 99.9375 93.5625)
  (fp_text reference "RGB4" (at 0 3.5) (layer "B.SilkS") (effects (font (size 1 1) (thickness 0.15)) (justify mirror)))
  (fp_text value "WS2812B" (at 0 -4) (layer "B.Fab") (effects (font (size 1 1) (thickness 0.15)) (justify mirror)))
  (pad "1" smd rect (at -2.45 1.65) (size 1.5 0.9) (layers "B.Cu" "B.Paste" "B.Mask") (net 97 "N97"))
  (pad "2" smd rect (at -2.45 -1.65) (size 1.5 0.9) (layers "B.Cu" "B.Paste" "B.Mask") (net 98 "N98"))
  (pad "3" smd rect (at 2.45 -1.65) (size 1.5 0.9) (layers "B.Cu" "B.Paste" "B.Mask") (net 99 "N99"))
  (pad "4" smd rect (at 2.45 1.65) (size 1.5 0.9) (layers "B.Cu" "B.Paste" "B.Mask") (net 82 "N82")))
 (gr_line (start 153.75 44.75) (end 93.75 44.75) (layer "Edge.Cuts") (width 0.2))
 (gr_arc (start 88.75 49.75) (mid 90.214466 46.214466) (end 93.75 44.75) (layer "Edge.Cuts") (width 0.2))
 (gr_line (start 88.75 49.75) (end 88.75 99.75) (layer "Edge.Cuts") (width 0.2))
 (gr_circle (center 155.078427 101.078427) (end 153.178427 101.078427) (layer "Edge.Cuts") (width 0.2) (fill none))
 (gr_arc (start 158.75 99.75) (mid 157.285534 103.285534) (end 153.75 104.75) (layer "Edge.Cuts") (width 0.2))
 (gr_arc (start 93.75 104.75) (mid 90.214466 103.285534) (end 88.75 99.75) (layer "Edge.Cuts") (width 0.2))
 (gr_circle (center 155.078427 48.421573) (end 153.178427 48.421573) (layer "Edge.Cuts") (width 0.2) (fill none))
 (gr_circle (center 92.421573 101.078427) (end 90.521573 101.078427) (layer "Edge.Cuts") (width 0.2) (fill none))
 (gr_line (start 93.75 104.75) (end 153.75 104.75) (layer "Edge.Cuts") (width 0.2))
 (gr_line (start 158.75 99.75) (end 158.75 49.75) (layer "Edge.Cuts") (width 0.2))
 (gr_circle (center 92.421573 48.421573) (end 90.521573 48.421573) (layer "Edge.Cuts") (width 0.2) (fill none))
 (gr_arc (start 153.75 44.75) (mid 157.285534 46.214466) (end 158.75 49.75) (layer "Edge.Cuts") (width 0.2))
 (segment (start 145.34 64.67) (end 145.34 84.0375) (width 0.2) (layer "B.Cu") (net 5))
 (segment (start 106.2125 86.2875) (end 108.0625 84.4375) (width 0.2) (layer "B.Cu") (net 15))
 (segment (start 111.84375 84.4375) (end 128.5125 84.4375) (width 0.2) (layer "B.Cu") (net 15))
 (segment (start 108.0625 84.4375) (end 111.84375 84.4375) (width 0.2) (layer "B.Cu") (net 15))
 (segment (start 96.6875 86.2875) (end 98.9375 84.0375) (width 0.2) (layer "B.Cu") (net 11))
 (segment (start 98.9375 84.0375) (end 128.5125 84.0375) (width 0.2) (layer "B.Cu") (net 11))
 (segment (start 115.7375 86.2875) (end 117.1875 84.8375) (width 0.2) (layer "B.Cu") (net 7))
 (segment (start 117.1875 84.8375) (end 118.9875 84.8375) (width 0.2) (layer "B.Cu") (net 7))
 (segment (start 118.9875 84.8375) (end 126.13125 84.8375) (width 0.2) (layer "B.Cu") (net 7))
 (segment (start 133.075 94.72) (end 133.275 94.92) (width 0.2) (layer "B.Cu") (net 3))
 (segment (start 133.075 92.2375) (end 133.075 94.72) (width 0.2) (layer "B.Cu") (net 3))
 (segment (start 134.675 92.902942) (end 135.723529 93.951471) (width 0.2) (layer "B.Cu") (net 37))
 (segment (start 134.675 92.2375) (end 134.675 92.902942) (width 0.2) (layer "B.Cu") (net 37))
 (segment (start 137.172058 95.4) (end 139.875 95.4) (width 0.2) (layer "B.Cu") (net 37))
 (segment (start 135.723529 93.951471) (end 137.172058 95.4) (width 0.2) (layer "B.Cu") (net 37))
 (via (at 138.275 97) (size 0.4) (drill 0.2) (layers "F.Cu" "B.Cu") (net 2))
 (segment (start 134.275 92.2375) (end 134.275 93.068628) (width 0.2) (layer "B.Cu") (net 2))
 (segment (start 138.206372 97) (end 138.275 97) (width 0.2) (layer "B.Cu") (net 2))
 (segment (start 134.740686 93.534314) (end 138.206372 97) (width 0.2) (layer "B.Cu") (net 2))
 (segment (start 134.275 93.068628) (end 134.740686 93.534314) (width 0.2) (layer "B.Cu") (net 2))
 (segment (start 136.875 96.234314) (end 136.875 97.8) (width 0.2) (layer "B.Cu") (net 38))
 (segment (start 133.875 92.2375) (end 133.875 93.234314) (width 0.2) (layer "B.Cu") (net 38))
 (segment (start 133.875 93.234314) (end 136.875 96.234314) (width 0.2) (layer "B.Cu") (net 38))
 (segment (start 133.475 92.2375) (end 133.475 93.4) (width 0.2) (layer "B.Cu") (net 39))
 (segment (start 133.475 93.4) (end 134.275 94.2) (width 0.2) (layer "B.Cu") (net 39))
 (segment (start 134.275 94.2) (end 134.275 94.92) (width 0.2) (layer "B.Cu") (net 39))
 (via (at 132.475 94.4) (size 0.4) (drill 0.2) (layers "F.Cu" "B.Cu") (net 1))
 (segment (start 132.275 94.92) (end 132.275 94.6) (width 0.2) (layer "B.Cu") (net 1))
 (segment (start 132.275 94.6) (end 132.475 94.4) (width 0.2) (layer "B.Cu") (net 1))
 (segment (start 132.675 94.52) (end 132.275 94.92) (width 0.2) (layer "B.Cu") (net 1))
 (segment (start 132.675 92.2375) (end 132.675 94.52) (width 0.2) (layer "B.Cu") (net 1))
 (segment (start 132.275 93.8) (end 130.875 95.2) (width 0.2) (layer "B.Cu") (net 40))
 (segment (start 130.875 95.2) (end 130.875 97.4) (width 0.2) (layer "B.Cu") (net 40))
 (segment (start 132.275 92.2375) (end 132.275 93.8) (width 0.2) (layer "B.Cu") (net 40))
 (segment (start 130.475 95.034315) (end 130.475 95.8) (width 0.2) (layer "B.Cu") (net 41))
 (segment (start 131.875 92.2375) (end 131.875 93.634314) (width 0.2) (layer "B.Cu") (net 41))
 (segment (start 131.875 93.634314) (end 130.475 95.034315) (width 0.2) (layer "B.Cu") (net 41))
 (segment (start 130.543629 94.4) (end 130.075 94.4) (width 0.2) (layer "B.Cu") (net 42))
 (segment (start 131.475 92.2375) (end 131.475 93.468628) (width 0.2) (layer "B.Cu") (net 42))
 (segment (start 131.475 93.468628) (end 130.543629 94.4) (width 0.2) (layer "B.Cu") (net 42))
 (segment (start 129.675 94.234315) (end 129.675 94.4) (width 0.2) (layer "B.Cu") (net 43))
 (segment (start 131.075 92.2375) (end 131.075 93.302943) (width 0.2) (layer "B.Cu") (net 43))
 (segment (start 130.377943 94) (end 129.909315 94) (width 0.2) (layer "B.Cu") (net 43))
 (segment (start 129.909315 94) (end 129.675 94.234315) (width 0.2) (layer "B.Cu") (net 43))
 (segment (start 131.075 93.302943) (end 130.377943 94) (width 0.2) (layer "B.Cu") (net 43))
 (segment (start 130.675 93.137257) (end 130.343628 93.468629) (width 0.2) (layer "B.Cu") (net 44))
 (segment (start 130.343628 93.468629) (end 130.212257 93.6) (width 0.2) (layer "B.Cu") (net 44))
 (segment (start 130.212257 93.6) (end 129.475 93.6) (width 0.2) (layer "B.Cu") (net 44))
 (segment (start 130.675 92.2375) (end 130.675 93.137257) (width 0.2) (layer "B.Cu") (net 44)))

